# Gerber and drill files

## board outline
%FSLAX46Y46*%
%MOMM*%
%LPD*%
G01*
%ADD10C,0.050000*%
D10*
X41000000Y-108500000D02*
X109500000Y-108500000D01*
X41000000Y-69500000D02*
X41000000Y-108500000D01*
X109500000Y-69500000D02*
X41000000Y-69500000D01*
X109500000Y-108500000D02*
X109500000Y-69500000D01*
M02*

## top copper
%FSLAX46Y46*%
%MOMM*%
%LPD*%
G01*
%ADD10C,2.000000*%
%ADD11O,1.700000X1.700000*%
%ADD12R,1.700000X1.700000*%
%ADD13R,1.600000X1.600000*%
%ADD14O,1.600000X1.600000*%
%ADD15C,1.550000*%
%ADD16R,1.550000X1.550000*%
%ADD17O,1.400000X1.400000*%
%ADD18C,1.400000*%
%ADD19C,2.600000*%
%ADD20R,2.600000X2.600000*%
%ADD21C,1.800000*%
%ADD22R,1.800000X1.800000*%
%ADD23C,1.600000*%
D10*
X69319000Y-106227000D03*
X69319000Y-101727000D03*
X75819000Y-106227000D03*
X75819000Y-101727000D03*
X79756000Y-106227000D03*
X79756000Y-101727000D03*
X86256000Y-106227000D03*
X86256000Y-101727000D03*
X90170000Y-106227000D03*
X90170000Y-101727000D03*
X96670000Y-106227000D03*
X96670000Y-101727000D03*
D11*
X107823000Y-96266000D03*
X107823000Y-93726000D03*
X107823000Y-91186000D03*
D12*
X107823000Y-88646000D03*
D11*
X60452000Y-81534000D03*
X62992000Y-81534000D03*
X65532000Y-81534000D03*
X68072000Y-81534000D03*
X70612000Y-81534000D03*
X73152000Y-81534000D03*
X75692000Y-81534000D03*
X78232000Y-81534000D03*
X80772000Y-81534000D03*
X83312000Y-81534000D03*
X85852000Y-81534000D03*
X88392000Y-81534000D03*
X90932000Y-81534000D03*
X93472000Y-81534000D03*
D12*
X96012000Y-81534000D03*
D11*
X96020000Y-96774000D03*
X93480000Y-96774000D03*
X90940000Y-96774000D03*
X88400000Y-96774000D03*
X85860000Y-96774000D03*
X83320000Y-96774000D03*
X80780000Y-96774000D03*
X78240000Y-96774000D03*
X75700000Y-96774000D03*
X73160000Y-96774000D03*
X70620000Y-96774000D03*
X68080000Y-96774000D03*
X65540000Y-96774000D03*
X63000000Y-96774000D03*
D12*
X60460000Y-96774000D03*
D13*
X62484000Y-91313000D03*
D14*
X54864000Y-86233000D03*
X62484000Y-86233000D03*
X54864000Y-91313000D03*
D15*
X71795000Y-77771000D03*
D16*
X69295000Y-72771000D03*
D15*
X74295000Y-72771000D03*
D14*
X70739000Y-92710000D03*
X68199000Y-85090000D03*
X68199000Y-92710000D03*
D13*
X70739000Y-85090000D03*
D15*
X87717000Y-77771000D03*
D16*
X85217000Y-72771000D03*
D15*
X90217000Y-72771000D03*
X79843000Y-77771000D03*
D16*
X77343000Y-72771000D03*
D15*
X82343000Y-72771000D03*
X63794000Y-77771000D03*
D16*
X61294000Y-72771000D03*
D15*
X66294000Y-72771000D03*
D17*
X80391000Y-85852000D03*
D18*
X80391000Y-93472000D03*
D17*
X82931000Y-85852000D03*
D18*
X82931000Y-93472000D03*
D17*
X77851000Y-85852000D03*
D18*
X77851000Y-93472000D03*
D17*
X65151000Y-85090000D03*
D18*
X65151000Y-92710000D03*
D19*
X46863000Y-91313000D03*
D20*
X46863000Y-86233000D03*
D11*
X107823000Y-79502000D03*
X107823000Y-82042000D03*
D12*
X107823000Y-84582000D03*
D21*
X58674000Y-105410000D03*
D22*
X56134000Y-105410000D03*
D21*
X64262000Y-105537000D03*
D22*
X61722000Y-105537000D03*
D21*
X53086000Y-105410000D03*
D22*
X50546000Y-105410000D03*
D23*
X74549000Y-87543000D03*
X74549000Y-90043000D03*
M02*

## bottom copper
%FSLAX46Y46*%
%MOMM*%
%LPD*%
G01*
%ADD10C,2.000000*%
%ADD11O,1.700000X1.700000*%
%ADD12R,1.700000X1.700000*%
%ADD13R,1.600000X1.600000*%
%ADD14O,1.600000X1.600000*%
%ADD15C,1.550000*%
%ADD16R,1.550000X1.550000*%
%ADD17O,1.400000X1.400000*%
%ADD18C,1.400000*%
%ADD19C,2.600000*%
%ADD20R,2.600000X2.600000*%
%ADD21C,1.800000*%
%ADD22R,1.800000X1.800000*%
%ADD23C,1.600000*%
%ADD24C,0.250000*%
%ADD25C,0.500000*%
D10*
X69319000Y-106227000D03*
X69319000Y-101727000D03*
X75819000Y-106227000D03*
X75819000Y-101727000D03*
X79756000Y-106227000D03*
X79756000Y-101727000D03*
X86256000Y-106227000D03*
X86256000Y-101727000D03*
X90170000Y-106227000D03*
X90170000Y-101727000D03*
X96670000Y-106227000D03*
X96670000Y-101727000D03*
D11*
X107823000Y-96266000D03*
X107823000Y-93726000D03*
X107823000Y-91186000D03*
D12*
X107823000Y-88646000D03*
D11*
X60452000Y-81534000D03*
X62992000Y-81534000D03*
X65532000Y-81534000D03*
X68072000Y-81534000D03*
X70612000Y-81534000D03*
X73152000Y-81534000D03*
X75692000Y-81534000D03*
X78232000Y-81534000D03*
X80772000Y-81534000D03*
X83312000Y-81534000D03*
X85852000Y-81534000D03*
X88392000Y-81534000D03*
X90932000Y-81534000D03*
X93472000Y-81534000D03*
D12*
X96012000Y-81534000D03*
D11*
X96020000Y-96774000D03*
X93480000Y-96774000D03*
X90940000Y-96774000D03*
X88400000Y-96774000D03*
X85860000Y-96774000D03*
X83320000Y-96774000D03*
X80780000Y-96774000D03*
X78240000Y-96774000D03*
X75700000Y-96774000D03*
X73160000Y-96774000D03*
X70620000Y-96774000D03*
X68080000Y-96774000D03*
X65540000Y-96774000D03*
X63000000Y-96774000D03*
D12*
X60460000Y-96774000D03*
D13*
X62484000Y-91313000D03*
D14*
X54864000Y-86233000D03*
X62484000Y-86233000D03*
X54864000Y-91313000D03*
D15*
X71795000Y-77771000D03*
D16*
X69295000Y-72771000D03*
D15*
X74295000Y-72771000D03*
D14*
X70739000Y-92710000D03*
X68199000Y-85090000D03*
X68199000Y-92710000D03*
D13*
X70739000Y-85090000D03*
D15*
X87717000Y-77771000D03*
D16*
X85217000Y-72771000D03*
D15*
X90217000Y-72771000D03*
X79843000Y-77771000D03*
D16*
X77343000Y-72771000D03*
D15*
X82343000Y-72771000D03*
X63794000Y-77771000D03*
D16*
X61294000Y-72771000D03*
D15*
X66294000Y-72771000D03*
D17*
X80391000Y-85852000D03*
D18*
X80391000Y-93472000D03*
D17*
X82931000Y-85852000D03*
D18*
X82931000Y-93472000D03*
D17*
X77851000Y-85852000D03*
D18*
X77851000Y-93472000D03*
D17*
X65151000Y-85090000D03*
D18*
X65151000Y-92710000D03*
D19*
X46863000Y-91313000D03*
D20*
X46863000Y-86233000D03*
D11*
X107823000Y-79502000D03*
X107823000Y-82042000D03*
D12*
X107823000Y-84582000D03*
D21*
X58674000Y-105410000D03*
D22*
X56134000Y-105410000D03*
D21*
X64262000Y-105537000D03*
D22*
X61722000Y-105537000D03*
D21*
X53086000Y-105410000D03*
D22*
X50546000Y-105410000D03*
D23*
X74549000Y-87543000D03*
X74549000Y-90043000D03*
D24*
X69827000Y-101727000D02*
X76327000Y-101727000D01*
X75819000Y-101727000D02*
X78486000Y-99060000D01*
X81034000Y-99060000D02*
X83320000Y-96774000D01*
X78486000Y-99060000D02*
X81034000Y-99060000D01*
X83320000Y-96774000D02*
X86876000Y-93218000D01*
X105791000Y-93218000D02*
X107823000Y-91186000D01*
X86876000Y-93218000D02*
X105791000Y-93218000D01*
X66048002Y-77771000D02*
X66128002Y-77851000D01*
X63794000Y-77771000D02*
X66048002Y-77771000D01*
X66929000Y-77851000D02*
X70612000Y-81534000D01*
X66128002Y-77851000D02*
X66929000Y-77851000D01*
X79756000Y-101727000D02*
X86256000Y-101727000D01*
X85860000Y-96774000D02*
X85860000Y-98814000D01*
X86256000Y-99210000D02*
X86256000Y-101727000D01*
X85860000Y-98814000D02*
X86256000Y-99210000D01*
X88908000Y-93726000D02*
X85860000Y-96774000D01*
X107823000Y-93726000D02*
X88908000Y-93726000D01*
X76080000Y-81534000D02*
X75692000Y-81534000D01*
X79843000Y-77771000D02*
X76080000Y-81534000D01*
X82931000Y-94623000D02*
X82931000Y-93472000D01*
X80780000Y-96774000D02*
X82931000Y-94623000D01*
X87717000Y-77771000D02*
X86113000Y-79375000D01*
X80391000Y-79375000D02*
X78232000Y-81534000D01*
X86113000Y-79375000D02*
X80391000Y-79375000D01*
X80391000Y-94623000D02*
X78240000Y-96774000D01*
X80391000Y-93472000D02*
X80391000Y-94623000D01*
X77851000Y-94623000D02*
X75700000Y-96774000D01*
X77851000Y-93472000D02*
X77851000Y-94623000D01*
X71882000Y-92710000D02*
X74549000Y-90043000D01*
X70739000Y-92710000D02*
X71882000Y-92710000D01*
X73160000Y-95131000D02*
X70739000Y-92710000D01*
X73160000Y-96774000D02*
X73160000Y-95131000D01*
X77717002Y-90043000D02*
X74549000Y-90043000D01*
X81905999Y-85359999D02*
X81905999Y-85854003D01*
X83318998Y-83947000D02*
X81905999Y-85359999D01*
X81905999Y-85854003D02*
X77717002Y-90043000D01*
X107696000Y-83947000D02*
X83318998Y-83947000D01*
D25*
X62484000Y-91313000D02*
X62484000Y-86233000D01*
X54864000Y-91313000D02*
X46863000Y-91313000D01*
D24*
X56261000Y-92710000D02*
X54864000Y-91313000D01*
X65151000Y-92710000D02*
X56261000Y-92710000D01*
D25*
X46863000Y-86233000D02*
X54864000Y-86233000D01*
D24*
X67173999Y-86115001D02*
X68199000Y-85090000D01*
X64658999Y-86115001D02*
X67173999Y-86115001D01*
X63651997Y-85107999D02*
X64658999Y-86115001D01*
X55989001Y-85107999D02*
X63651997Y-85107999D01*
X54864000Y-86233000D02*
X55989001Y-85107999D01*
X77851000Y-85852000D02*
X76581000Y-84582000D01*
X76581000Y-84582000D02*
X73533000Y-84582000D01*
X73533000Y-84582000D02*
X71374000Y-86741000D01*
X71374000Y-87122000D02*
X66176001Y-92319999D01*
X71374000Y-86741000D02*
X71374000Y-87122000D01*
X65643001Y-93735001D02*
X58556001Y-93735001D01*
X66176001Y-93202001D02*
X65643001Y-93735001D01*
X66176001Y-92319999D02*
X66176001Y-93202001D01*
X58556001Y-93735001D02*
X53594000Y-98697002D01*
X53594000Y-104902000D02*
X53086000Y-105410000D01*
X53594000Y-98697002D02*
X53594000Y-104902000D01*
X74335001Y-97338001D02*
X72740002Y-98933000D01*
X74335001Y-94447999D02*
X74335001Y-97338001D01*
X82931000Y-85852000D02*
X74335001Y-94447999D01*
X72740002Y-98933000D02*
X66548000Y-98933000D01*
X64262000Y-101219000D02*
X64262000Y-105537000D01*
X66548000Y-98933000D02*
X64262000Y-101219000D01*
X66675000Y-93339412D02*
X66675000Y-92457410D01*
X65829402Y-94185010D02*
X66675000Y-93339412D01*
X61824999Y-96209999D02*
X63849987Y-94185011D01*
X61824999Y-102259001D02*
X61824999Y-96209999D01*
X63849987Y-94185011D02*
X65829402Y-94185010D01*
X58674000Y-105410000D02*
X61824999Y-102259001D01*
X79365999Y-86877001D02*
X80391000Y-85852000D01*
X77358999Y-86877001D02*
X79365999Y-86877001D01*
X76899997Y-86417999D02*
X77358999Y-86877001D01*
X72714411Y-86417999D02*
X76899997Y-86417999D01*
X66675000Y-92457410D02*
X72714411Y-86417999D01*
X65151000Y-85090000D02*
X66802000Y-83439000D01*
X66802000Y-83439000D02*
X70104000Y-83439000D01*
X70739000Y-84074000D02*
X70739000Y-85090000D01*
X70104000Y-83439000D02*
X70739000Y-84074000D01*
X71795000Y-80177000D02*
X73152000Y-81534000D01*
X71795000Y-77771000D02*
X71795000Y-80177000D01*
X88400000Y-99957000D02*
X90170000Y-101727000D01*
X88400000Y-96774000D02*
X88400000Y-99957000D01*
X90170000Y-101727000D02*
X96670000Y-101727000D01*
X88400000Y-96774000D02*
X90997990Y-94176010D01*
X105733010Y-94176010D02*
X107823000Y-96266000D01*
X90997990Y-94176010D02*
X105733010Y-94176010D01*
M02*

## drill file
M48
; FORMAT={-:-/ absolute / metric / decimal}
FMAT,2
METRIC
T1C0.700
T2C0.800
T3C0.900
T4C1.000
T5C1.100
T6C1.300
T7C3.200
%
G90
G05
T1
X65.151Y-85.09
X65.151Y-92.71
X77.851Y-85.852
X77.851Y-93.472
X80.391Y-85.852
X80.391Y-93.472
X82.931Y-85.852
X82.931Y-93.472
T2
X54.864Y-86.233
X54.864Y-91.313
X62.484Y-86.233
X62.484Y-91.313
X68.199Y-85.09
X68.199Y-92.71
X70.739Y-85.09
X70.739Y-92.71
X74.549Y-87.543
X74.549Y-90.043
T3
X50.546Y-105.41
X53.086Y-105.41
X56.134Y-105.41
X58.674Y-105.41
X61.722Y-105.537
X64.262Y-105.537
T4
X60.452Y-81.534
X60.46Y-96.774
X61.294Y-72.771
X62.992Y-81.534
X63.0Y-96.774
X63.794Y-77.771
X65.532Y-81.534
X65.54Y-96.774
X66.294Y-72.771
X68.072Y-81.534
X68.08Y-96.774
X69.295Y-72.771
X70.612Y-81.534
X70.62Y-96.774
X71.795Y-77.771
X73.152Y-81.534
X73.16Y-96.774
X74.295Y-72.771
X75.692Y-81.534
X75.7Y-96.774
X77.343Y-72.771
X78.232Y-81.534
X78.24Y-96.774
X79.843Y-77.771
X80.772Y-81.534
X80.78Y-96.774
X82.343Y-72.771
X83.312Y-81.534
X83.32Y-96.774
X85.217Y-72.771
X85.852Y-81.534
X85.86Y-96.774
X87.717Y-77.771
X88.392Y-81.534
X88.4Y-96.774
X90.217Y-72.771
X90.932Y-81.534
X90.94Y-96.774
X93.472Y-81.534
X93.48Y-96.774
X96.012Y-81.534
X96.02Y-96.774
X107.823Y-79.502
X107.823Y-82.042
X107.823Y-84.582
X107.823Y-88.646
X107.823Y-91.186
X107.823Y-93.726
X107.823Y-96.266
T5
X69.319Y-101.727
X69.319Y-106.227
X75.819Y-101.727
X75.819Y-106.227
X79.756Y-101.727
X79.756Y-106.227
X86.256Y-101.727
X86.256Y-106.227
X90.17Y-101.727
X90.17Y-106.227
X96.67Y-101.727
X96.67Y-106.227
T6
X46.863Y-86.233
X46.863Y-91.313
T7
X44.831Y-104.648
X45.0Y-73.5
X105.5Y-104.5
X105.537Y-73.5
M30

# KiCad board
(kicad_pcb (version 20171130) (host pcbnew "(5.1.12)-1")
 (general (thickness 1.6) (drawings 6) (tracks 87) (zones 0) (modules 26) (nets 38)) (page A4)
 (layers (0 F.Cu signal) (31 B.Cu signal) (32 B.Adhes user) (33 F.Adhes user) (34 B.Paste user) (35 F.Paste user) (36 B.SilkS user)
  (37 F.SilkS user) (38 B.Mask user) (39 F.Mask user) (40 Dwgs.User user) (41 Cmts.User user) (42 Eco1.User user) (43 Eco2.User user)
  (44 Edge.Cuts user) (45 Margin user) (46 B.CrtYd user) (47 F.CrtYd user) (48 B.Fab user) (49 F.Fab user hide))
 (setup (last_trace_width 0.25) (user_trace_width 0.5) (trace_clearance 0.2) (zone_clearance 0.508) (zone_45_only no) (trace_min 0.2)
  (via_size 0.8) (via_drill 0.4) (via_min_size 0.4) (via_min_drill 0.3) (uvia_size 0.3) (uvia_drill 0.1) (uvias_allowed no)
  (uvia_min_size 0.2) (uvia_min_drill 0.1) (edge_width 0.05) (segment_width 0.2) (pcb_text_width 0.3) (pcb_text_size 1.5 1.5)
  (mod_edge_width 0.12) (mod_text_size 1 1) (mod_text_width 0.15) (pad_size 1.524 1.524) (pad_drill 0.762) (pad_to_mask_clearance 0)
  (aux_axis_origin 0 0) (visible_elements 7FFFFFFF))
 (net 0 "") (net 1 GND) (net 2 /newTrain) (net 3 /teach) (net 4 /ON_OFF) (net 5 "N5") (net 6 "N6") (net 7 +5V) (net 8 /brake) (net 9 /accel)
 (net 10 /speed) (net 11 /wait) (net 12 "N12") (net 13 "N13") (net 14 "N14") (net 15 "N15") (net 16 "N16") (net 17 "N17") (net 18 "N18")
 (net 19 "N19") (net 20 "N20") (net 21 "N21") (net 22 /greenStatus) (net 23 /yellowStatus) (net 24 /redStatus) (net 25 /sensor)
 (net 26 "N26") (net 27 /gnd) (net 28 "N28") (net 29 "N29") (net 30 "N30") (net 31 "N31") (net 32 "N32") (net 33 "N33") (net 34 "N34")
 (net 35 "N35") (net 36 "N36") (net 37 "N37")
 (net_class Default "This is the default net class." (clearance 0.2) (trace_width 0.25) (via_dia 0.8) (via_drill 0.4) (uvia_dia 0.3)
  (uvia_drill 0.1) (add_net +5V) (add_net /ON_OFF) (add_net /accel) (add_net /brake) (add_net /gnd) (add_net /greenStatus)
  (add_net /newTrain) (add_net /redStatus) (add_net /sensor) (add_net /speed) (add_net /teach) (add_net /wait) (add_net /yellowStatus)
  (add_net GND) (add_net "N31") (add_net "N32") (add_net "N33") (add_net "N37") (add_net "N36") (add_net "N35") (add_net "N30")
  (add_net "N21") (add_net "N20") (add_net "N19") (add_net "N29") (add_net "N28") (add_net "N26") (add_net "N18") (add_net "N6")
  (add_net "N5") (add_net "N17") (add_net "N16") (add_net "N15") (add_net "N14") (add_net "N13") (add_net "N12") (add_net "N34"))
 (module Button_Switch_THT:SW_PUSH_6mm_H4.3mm (layer F.Cu) (at 75.819 106.227 180)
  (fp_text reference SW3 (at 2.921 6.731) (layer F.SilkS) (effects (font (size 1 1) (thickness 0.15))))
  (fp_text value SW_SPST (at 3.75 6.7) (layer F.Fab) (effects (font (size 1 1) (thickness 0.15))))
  (pad 1 thru_hole circle (at 6.5 0 270) (size 2 2) (drill 1.1) (layers *.Cu *.Mask) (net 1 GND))
  (pad 2 thru_hole circle (at 6.5 4.5 270) (size 2 2) (drill 1.1) (layers *.Cu *.Mask) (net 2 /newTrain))
  (pad 1 thru_hole circle (at 0 0 270) (size 2 2) (drill 1.1) (layers *.Cu *.Mask) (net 1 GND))
  (pad 2 thru_hole circle (at 0 4.5 270) (size 2 2) (drill 1.1) (layers *.Cu *.Mask) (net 2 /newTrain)))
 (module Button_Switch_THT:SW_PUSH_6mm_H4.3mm (layer F.Cu) (at 86.256 106.227 180)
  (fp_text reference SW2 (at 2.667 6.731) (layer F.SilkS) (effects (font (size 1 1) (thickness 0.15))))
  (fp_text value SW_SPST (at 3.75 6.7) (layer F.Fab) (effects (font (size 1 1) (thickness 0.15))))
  (pad 1 thru_hole circle (at 6.5 0 270) (size 2 2) (drill 1.1) (layers *.Cu *.Mask) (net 1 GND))
  (pad 2 thru_hole circle (at 6.5 4.5 270) (size 2 2) (drill 1.1) (layers *.Cu *.Mask) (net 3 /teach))
  (pad 1 thru_hole circle (at 0 0 270) (size 2 2) (drill 1.1) (layers *.Cu *.Mask) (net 1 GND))
  (pad 2 thru_hole circle (at 0 4.5 270) (size 2 2) (drill 1.1) (layers *.Cu *.Mask) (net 3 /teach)))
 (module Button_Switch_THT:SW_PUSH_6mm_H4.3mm (layer F.Cu) (at 96.67 106.227 180)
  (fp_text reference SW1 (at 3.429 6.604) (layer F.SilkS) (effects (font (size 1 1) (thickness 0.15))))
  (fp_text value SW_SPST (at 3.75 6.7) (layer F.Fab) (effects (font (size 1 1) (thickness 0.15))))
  (pad 1 thru_hole circle (at 6.5 0 270) (size 2 2) (drill 1.1) (layers *.Cu *.Mask) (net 1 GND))
  (pad 2 thru_hole circle (at 6.5 4.5 270) (size 2 2) (drill 1.1) (layers *.Cu *.Mask) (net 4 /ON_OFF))
  (pad 1 thru_hole circle (at 0 0 270) (size 2 2) (drill 1.1) (layers *.Cu *.Mask) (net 1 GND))
  (pad 2 thru_hole circle (at 0 4.5 270) (size 2 2) (drill 1.1) (layers *.Cu *.Mask) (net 4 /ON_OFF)))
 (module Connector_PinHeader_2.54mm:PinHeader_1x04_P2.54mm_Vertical (layer F.Cu) (at 107.823 88.646)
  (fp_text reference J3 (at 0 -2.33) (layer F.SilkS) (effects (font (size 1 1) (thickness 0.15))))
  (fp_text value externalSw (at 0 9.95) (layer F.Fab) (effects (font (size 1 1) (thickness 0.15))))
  (pad 4 thru_hole oval (at 0 7.62) (size 1.7 1.7) (drill 1) (layers *.Cu *.Mask) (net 4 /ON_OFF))
  (pad 3 thru_hole oval (at 0 5.08) (size 1.7 1.7) (drill 1) (layers *.Cu *.Mask) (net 3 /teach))
  (pad 2 thru_hole oval (at 0 2.54) (size 1.7 1.7) (drill 1) (layers *.Cu *.Mask) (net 2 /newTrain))
  (pad 1 thru_hole rect (at 0 0) (size 1.7 1.7) (drill 1) (layers *.Cu *.Mask) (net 1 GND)))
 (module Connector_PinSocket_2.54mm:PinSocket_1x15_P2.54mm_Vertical (layer F.Cu) (at 96.012 81.534 270)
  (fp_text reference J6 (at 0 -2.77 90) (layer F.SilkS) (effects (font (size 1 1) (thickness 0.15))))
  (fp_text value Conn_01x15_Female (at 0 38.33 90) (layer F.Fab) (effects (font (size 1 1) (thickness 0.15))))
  (pad 15 thru_hole oval (at 0 35.56 270) (size 1.7 1.7) (drill 1) (layers *.Cu *.Mask) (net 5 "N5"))
  (pad 14 thru_hole oval (at 0 33.02 270) (size 1.7 1.7) (drill 1) (layers *.Cu *.Mask) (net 1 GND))
  (pad 13 thru_hole oval (at 0 30.48 270) (size 1.7 1.7) (drill 1) (layers *.Cu *.Mask) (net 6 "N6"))
  (pad 12 thru_hole oval (at 0 27.94 270) (size 1.7 1.7) (drill 1) (layers *.Cu *.Mask) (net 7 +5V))
  (pad 11 thru_hole oval (at 0 25.4 270) (size 1.7 1.7) (drill 1) (layers *.Cu *.Mask) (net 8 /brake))
  (pad 10 thru_hole oval (at 0 22.86 270) (size 1.7 1.7) (drill 1) (layers *.Cu *.Mask) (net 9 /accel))
  (pad 9 thru_hole oval (at 0 20.32 270) (size 1.7 1.7) (drill 1) (layers *.Cu *.Mask) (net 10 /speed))
  (pad 8 thru_hole oval (at 0 17.78 270) (size 1.7 1.7) (drill 1) (layers *.Cu *.Mask) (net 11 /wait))
  (pad 7 thru_hole oval (at 0 15.24 270) (size 1.7 1.7) (drill 1) (layers *.Cu *.Mask) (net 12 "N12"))
  (pad 6 thru_hole oval (at 0 12.7 270) (size 1.7 1.7) (drill 1) (layers *.Cu *.Mask) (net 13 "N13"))
  (pad 5 thru_hole oval (at 0 10.16 270) (size 1.7 1.7) (drill 1) (layers *.Cu *.Mask) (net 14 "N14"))
  (pad 4 thru_hole oval (at 0 7.62 270) (size 1.7 1.7) (drill 1) (layers *.Cu *.Mask) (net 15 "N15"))
  (pad 3 thru_hole oval (at 0 5.08 270) (size 1.7 1.7) (drill 1) (layers *.Cu *.Mask) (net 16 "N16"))
  (pad 2 thru_hole oval (at 0 2.54 270) (size 1.7 1.7) (drill 1) (layers *.Cu *.Mask) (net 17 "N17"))
  (pad 1 thru_hole rect (at 0 0 270) (size 1.7 1.7) (drill 1) (layers *.Cu *.Mask) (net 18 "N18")))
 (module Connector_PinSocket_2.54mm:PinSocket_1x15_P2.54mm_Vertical (layer F.Cu) (at 60.46 96.774 90)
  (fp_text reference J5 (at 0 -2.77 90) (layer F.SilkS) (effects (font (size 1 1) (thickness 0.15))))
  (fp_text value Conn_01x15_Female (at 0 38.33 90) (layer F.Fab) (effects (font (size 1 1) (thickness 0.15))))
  (pad 15 thru_hole oval (at 0 35.56 90) (size 1.7 1.7) (drill 1) (layers *.Cu *.Mask) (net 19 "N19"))
  (pad 14 thru_hole oval (at 0 33.02 90) (size 1.7 1.7) (drill 1) (layers *.Cu *.Mask) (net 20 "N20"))
  (pad 13 thru_hole oval (at 0 30.48 90) (size 1.7 1.7) (drill 1) (layers *.Cu *.Mask) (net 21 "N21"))
  (pad 12 thru_hole oval (at 0 27.94 90) (size 1.7 1.7) (drill 1) (layers *.Cu *.Mask) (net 4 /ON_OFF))
  (pad 11 thru_hole oval (at 0 25.4 90) (size 1.7 1.7) (drill 1) (layers *.Cu *.Mask) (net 3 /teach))
  (pad 10 thru_hole oval (at 0 22.86 90) (size 1.7 1.7) (drill 1) (layers *.Cu *.Mask) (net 2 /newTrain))
  (pad 9 thru_hole oval (at 0 20.32 90) (size 1.7 1.7) (drill 1) (layers *.Cu *.Mask) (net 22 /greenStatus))
  (pad 8 thru_hole oval (at 0 17.78 90) (size 1.7 1.7) (drill 1) (layers *.Cu *.Mask) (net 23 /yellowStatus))
  (pad 7 thru_hole oval (at 0 15.24 90) (size 1.7 1.7) (drill 1) (layers *.Cu *.Mask) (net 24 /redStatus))
  (pad 6 thru_hole oval (at 0 12.7 90) (size 1.7 1.7) (drill 1) (layers *.Cu *.Mask) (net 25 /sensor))
  (pad 5 thru_hole oval (at 0 10.16 90) (size 1.7 1.7) (drill 1) (layers *.Cu *.Mask) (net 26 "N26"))
  (pad 4 thru_hole oval (at 0 7.62 90) (size 1.7 1.7) (drill 1) (layers *.Cu *.Mask) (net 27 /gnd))
  (pad 3 thru_hole oval (at 0 5.08 90) (size 1.7 1.7) (drill 1) (layers *.Cu *.Mask) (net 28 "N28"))
  (pad 2 thru_hole oval (at 0 2.54 90) (size 1.7 1.7) (drill 1) (layers *.Cu *.Mask) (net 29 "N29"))
  (pad 1 thru_hole rect (at 0 0 90) (size 1.7 1.7) (drill 1) (layers *.Cu *.Mask) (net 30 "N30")))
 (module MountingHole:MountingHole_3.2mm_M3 (layer F.Cu) (at 44.831 104.648)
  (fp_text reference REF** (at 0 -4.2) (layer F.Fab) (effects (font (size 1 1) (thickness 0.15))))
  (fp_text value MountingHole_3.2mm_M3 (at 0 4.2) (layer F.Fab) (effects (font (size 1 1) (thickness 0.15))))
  (pad 1 np_thru_hole circle (at 0 0) (size 3.2 3.2) (drill 3.2) (layers *.Cu *.Mask)))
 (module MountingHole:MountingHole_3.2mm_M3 (layer F.Cu) (at 45 73.5)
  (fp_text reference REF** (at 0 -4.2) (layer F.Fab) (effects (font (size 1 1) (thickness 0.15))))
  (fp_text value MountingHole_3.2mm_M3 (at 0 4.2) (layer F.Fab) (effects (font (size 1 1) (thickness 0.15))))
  (pad 1 np_thru_hole circle (at 0 0) (size 3.2 3.2) (drill 3.2) (layers *.Cu *.Mask)))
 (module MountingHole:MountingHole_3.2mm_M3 (layer F.Cu) (at 105.537 73.5)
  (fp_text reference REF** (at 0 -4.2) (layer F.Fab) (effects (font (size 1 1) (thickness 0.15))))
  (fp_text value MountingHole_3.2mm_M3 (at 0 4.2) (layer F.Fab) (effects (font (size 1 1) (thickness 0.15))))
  (pad 1 np_thru_hole circle (at 0 0) (size 3.2 3.2) (drill 3.2) (layers *.Cu *.Mask)))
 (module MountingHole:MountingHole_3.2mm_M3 (layer F.Cu) (at 105.5 104.5)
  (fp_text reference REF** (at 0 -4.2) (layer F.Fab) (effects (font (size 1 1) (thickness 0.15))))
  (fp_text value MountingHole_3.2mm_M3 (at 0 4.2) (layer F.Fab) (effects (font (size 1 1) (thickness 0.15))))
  (pad 1 np_thru_hole circle (at 0 0) (size 3.2 3.2) (drill 3.2) (layers *.Cu *.Mask)))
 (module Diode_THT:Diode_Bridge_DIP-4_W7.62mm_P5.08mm (layer F.Cu) (at 62.484 91.313 180)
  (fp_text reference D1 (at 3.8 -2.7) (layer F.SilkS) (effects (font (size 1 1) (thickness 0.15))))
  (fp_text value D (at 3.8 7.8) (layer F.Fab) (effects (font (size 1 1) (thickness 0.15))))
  (pad 1 thru_hole rect (at 0 0 180) (size 1.6 1.6) (drill 0.8) (layers *.Cu *.Mask) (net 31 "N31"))
  (pad 3 thru_hole oval (at 7.62 5.08 180) (size 1.6 1.6) (drill 0.8) (layers *.Cu *.Mask) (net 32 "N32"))
  (pad 2 thru_hole oval (at 0 5.08 180) (size 1.6 1.6) (drill 0.8) (layers *.Cu *.Mask) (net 31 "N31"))
  (pad 4 thru_hole oval (at 7.62 0 180) (size 1.6 1.6) (drill 0.8) (layers *.Cu *.Mask) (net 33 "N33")))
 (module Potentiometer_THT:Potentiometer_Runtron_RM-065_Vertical (layer F.Cu) (at 69.295 72.771)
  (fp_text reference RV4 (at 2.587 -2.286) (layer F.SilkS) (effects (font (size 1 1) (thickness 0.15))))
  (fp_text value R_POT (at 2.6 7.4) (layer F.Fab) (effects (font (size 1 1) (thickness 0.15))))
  (pad 2 thru_hole circle (at 2.5 5) (size 1.55 1.55) (drill 1) (layers *.Cu *.Mask) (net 9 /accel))
  (pad 1 thru_hole rect (at 0 0) (size 1.55 1.55) (drill 1) (layers *.Cu *.Mask) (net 1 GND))
  (pad 3 thru_hole circle (at 5 0) (size 1.55 1.55) (drill 1) (layers *.Cu *.Mask) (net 7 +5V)))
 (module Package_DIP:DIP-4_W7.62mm (layer F.Cu) (at 70.739 85.09 270)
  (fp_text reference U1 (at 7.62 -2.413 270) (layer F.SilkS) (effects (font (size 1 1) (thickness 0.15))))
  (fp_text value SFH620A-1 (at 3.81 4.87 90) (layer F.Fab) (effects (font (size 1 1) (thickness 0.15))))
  (pad 4 thru_hole oval (at 7.62 0 270) (size 1.6 1.6) (drill 0.8) (layers *.Cu *.Mask) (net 25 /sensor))
  (pad 2 thru_hole oval (at 0 2.54 270) (size 1.6 1.6) (drill 0.8) (layers *.Cu *.Mask) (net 32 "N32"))
  (pad 3 thru_hole oval (at 7.62 2.54 270) (size 1.6 1.6) (drill 0.8) (layers *.Cu *.Mask) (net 1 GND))
  (pad 1 thru_hole rect (at 0 0 270) (size 1.6 1.6) (drill 0.8) (layers *.Cu *.Mask) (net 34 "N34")))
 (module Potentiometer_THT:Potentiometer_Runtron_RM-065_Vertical (layer F.Cu) (at 85.217 72.771)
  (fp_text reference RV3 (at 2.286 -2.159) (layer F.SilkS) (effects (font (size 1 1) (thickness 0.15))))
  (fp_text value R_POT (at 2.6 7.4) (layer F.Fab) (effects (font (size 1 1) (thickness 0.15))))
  (pad 2 thru_hole circle (at 2.5 5) (size 1.55 1.55) (drill 1) (layers *.Cu *.Mask) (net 11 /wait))
  (pad 1 thru_hole rect (at 0 0) (size 1.55 1.55) (drill 1) (layers *.Cu *.Mask) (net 1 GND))
  (pad 3 thru_hole circle (at 5 0) (size 1.55 1.55) (drill 1) (layers *.Cu *.Mask) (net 7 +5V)))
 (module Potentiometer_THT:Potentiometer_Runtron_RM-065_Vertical (layer F.Cu) (at 77.343 72.771)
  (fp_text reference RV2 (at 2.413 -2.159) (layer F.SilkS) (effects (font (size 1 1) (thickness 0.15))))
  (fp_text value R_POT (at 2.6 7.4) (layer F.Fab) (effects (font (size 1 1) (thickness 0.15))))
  (pad 2 thru_hole circle (at 2.5 5) (size 1.55 1.55) (drill 1) (layers *.Cu *.Mask) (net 10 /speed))
  (pad 1 thru_hole rect (at 0 0) (size 1.55 1.55) (drill 1) (layers *.Cu *.Mask) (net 1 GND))
  (pad 3 thru_hole circle (at 5 0) (size 1.55 1.55) (drill 1) (layers *.Cu *.Mask) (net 7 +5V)))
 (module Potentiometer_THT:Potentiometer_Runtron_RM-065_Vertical (layer F.Cu) (at 61.294 72.771)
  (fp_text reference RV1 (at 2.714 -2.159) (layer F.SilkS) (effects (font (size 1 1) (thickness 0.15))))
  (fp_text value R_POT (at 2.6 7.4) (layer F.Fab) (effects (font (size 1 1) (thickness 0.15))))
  (pad 2 thru_hole circle (at 2.5 5) (size 1.55 1.55) (drill 1) (layers *.Cu *.Mask) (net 8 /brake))
  (pad 1 thru_hole rect (at 0 0) (size 1.55 1.55) (drill 1) (layers *.Cu *.Mask) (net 1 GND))
  (pad 3 thru_hole circle (at 5 0) (size 1.55 1.55) (drill 1) (layers *.Cu *.Mask) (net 7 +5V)))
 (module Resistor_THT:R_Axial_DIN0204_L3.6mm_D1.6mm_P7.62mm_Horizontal (layer F.Cu) (at 80.391 93.472 90)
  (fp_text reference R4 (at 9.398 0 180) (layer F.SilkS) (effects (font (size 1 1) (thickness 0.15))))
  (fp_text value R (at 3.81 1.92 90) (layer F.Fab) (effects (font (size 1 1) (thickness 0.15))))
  (pad 2 thru_hole oval (at 7.62 0 90) (size 1.4 1.4) (drill 0.7) (layers *.Cu *.Mask) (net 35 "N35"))
  (pad 1 thru_hole circle (at 0 0 90) (size 1.4 1.4) (drill 0.7) (layers *.Cu *.Mask) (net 23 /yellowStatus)))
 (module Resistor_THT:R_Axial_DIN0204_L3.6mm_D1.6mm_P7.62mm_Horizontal (layer F.Cu) (at 82.931 93.472 90)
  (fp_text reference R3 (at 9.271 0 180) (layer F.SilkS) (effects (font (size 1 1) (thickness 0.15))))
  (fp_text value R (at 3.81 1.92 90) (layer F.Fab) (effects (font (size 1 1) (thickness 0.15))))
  (pad 2 thru_hole oval (at 7.62 0 90) (size 1.4 1.4) (drill 0.7) (layers *.Cu *.Mask) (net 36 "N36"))
  (pad 1 thru_hole circle (at 0 0 90) (size 1.4 1.4) (drill 0.7) (layers *.Cu *.Mask) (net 22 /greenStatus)))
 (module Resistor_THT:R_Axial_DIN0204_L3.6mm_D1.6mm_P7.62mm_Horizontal (layer F.Cu) (at 77.851 93.472 90)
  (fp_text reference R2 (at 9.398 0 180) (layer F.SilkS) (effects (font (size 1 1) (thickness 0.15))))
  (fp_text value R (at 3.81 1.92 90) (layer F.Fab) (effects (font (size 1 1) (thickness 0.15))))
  (pad 2 thru_hole oval (at 7.62 0 90) (size 1.4 1.4) (drill 0.7) (layers *.Cu *.Mask) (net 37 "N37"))
  (pad 1 thru_hole circle (at 0 0 90) (size 1.4 1.4) (drill 0.7) (layers *.Cu *.Mask) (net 24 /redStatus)))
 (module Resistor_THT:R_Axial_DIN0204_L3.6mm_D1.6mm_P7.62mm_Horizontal (layer F.Cu) (at 65.151 92.71 90)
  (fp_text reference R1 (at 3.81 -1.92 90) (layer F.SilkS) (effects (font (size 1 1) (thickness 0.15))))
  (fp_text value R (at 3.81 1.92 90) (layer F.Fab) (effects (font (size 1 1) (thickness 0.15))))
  (pad 2 thru_hole oval (at 7.62 0 90) (size 1.4 1.4) (drill 0.7) (layers *.Cu *.Mask) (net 34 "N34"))
  (pad 1 thru_hole circle (at 0 0 90) (size 1.4 1.4) (drill 0.7) (layers *.Cu *.Mask) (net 33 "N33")))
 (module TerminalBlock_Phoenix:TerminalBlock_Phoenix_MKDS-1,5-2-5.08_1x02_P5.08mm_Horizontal (layer F.Cu) (at 46.863 86.233 270)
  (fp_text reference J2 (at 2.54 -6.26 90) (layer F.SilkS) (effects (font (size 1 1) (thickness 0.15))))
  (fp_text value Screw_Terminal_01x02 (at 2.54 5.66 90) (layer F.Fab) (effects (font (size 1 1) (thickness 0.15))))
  (pad 2 thru_hole circle (at 5.08 0 270) (size 2.6 2.6) (drill 1.3) (layers *.Cu *.Mask) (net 33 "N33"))
  (pad 1 thru_hole rect (at 0 0 270) (size 2.6 2.6) (drill 1.3) (layers *.Cu *.Mask) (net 32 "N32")))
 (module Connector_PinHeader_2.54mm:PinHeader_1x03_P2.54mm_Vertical (layer F.Cu) (at 107.823 84.582 180)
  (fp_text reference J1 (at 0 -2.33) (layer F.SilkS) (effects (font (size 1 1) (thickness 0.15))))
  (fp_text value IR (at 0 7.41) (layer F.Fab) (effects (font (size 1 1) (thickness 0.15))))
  (pad 3 thru_hole oval (at 0 5.08 180) (size 1.7 1.7) (drill 1) (layers *.Cu *.Mask) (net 1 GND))
  (pad 2 thru_hole oval (at 0 2.54 180) (size 1.7 1.7) (drill 1) (layers *.Cu *.Mask) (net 7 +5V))
  (pad 1 thru_hole rect (at 0 0 180) (size 1.7 1.7) (drill 1) (layers *.Cu *.Mask) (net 25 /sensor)))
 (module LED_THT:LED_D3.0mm (layer F.Cu) (at 56.134 105.41)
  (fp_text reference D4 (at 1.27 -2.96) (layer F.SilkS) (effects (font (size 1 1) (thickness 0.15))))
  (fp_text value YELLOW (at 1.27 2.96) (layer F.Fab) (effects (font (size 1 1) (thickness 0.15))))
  (pad 2 thru_hole circle (at 2.54 0) (size 1.8 1.8) (drill 0.9) (layers *.Cu *.Mask) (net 35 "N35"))
  (pad 1 thru_hole rect (at 0 0) (size 1.8 1.8) (drill 0.9) (layers *.Cu *.Mask) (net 1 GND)))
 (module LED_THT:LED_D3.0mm (layer F.Cu) (at 61.722 105.537)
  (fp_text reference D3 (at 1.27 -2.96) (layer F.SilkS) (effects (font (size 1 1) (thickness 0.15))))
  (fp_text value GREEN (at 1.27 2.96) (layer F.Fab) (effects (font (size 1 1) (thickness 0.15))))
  (pad 2 thru_hole circle (at 2.54 0) (size 1.8 1.8) (drill 0.9) (layers *.Cu *.Mask) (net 36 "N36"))
  (pad 1 thru_hole rect (at 0 0) (size 1.8 1.8) (drill 0.9) (layers *.Cu *.Mask) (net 1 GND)))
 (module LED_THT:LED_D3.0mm (layer F.Cu) (at 50.546 105.41)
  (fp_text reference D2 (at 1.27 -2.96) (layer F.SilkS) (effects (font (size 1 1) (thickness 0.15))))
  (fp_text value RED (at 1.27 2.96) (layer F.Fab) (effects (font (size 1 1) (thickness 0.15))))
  (pad 2 thru_hole circle (at 2.54 0) (size 1.8 1.8) (drill 0.9) (layers *.Cu *.Mask) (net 37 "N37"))
  (pad 1 thru_hole rect (at 0 0) (size 1.8 1.8) (drill 0.9) (layers *.Cu *.Mask) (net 1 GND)))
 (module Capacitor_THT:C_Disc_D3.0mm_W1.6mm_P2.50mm (layer F.Cu) (at 74.549 90.043 90)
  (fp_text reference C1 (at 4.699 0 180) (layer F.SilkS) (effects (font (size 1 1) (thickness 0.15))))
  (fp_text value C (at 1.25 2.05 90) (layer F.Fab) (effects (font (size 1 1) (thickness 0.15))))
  (pad 2 thru_hole circle (at 2.5 0 90) (size 1.6 1.6) (drill 0.8) (layers *.Cu *.Mask) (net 1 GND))
  (pad 1 thru_hole circle (at 0 0 90) (size 1.6 1.6) (drill 0.8) (layers *.Cu *.Mask) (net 25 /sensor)))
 (gr_line (start 41 108.5) (end 109.5 108.5) (layer Edge.Cuts) (width 0.05))
 (gr_line (start 41 69.5) (end 41 108.5) (layer Edge.Cuts) (width 0.05))
 (gr_line (start 109.5 69.5) (end 41 69.5) (layer Edge.Cuts) (width 0.05))
 (gr_line (start 109.5 108.5) (end 109.5 69.5) (layer Edge.Cuts) (width 0.05))
 (segment (start 69.827 101.727) (end 76.327 101.727) (width 0.25) (layer B.Cu) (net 2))
 (segment (start 75.819 101.727) (end 78.486 99.06) (width 0.25) (layer B.Cu) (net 2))
 (segment (start 81.034 99.06) (end 83.32 96.774) (width 0.25) (layer B.Cu) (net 2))
 (segment (start 78.486 99.06) (end 81.034 99.06) (width 0.25) (layer B.Cu) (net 2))
 (segment (start 83.32 96.774) (end 86.876 93.218) (width 0.25) (layer B.Cu) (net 2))
 (segment (start 105.791 93.218) (end 107.823 91.186) (width 0.25) (layer B.Cu) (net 2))
 (segment (start 86.876 93.218) (end 105.791 93.218) (width 0.25) (layer B.Cu) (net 2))
 (segment (start 66.048002 77.771) (end 66.128002 77.851) (width 0.25) (layer B.Cu) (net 8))
 (segment (start 63.794 77.771) (end 66.048002 77.771) (width 0.25) (layer B.Cu) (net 8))
 (segment (start 66.929 77.851) (end 70.612 81.534) (width 0.25) (layer B.Cu) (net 8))
 (segment (start 66.128002 77.851) (end 66.929 77.851) (width 0.25) (layer B.Cu) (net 8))
 (segment (start 79.756 101.727) (end 86.256 101.727) (width 0.25) (layer B.Cu) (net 3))
 (segment (start 85.86 96.774) (end 85.86 98.814) (width 0.25) (layer B.Cu) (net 3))
 (segment (start 86.256 99.21) (end 86.256 101.727) (width 0.25) (layer B.Cu) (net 3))
 (segment (start 85.86 98.814) (end 86.256 99.21) (width 0.25) (layer B.Cu) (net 3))
 (segment (start 88.908 93.726) (end 85.86 96.774) (width 0.25) (layer B.Cu) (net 3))
 (segment (start 107.823 93.726) (end 88.908 93.726) (width 0.25) (layer B.Cu) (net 3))
 (segment (start 76.08 81.534) (end 75.692 81.534) (width 0.25) (layer B.Cu) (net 10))
 (segment (start 79.843 77.771) (end 76.08 81.534) (width 0.25) (layer B.Cu) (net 10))
 (segment (start 82.931 94.623) (end 82.931 93.472) (width 0.25) (layer B.Cu) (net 22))
 (segment (start 80.78 96.774) (end 82.931 94.623) (width 0.25) (layer B.Cu) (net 22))
 (segment (start 87.717 77.771) (end 86.113 79.375) (width 0.25) (layer B.Cu) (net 11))
 (segment (start 80.391 79.375) (end 78.232 81.534) (width 0.25) (layer B.Cu) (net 11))
 (segment (start 86.113 79.375) (end 80.391 79.375) (width 0.25) (layer B.Cu) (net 11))
 (segment (start 80.391 94.623) (end 78.24 96.774) (width 0.25) (layer B.Cu) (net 23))
 (segment (start 80.391 93.472) (end 80.391 94.623) (width 0.25) (layer B.Cu) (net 23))
 (segment (start 77.851 94.623) (end 75.7 96.774) (width 0.25) (layer B.Cu) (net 24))
 (segment (start 77.851 93.472) (end 77.851 94.623) (width 0.25) (layer B.Cu) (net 24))
 (segment (start 71.882 92.71) (end 74.549 90.043) (width 0.25) (layer B.Cu) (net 25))
 (segment (start 70.739 92.71) (end 71.882 92.71) (width 0.25) (layer B.Cu) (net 25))
 (segment (start 73.16 95.131) (end 70.739 92.71) (width 0.25) (layer B.Cu) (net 25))
 (segment (start 73.16 96.774) (end 73.16 95.131) (width 0.25) (layer B.Cu) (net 25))
 (segment (start 77.717002 90.043) (end 74.549 90.043) (width 0.25) (layer B.Cu) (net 25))
 (segment (start 81.905999 85.359999) (end 81.905999 85.854003) (width 0.25) (layer B.Cu) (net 25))
 (segment (start 83.318998 83.947) (end 81.905999 85.359999) (width 0.25) (layer B.Cu) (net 25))
 (segment (start 81.905999 85.854003) (end 77.717002 90.043) (width 0.25) (layer B.Cu) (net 25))
 (segment (start 107.696 83.947) (end 83.318998 83.947) (width 0.25) (layer B.Cu) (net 25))
 (segment (start 62.484 91.313) (end 62.484 86.233) (width 0.5) (layer B.Cu) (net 31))
 (segment (start 54.864 91.313) (end 46.863 91.313) (width 0.5) (layer B.Cu) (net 33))
 (segment (start 56.261 92.71) (end 54.864 91.313) (width 0.25) (layer B.Cu) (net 33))
 (segment (start 65.151 92.71) (end 56.261 92.71) (width 0.25) (layer B.Cu) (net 33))
 (segment (start 46.863 86.233) (end 54.864 86.233) (width 0.5) (layer B.Cu) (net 32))
 (segment (start 67.173999 86.115001) (end 68.199 85.09) (width 0.25) (layer B.Cu) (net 32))
 (segment (start 64.658999 86.115001) (end 67.173999 86.115001) (width 0.25) (layer B.Cu) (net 32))
 (segment (start 63.651997 85.107999) (end 64.658999 86.115001) (width 0.25) (layer B.Cu) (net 32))
 (segment (start 55.989001 85.107999) (end 63.651997 85.107999) (width 0.25) (layer B.Cu) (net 32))
 (segment (start 54.864 86.233) (end 55.989001 85.107999) (width 0.25) (layer B.Cu) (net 32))
 (segment (start 77.851 85.852) (end 76.581 84.582) (width 0.25) (layer B.Cu) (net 37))
 (segment (start 76.581 84.582) (end 73.533 84.582) (width 0.25) (layer B.Cu) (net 37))
 (segment (start 73.533 84.582) (end 71.374 86.741) (width 0.25) (layer B.Cu) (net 37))
 (segment (start 71.374 87.122) (end 66.176001 92.319999) (width 0.25) (layer B.Cu) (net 37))
 (segment (start 71.374 86.741) (end 71.374 87.122) (width 0.25) (layer B.Cu) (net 37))
 (segment (start 65.643001 93.735001) (end 58.556001 93.735001) (width 0.25) (layer B.Cu) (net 37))
 (segment (start 66.176001 93.202001) (end 65.643001 93.735001) (width 0.25) (layer B.Cu) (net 37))
 (segment (start 66.176001 92.319999) (end 66.176001 93.202001) (width 0.25) (layer B.Cu) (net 37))
 (segment (start 58.556001 93.735001) (end 53.594 98.697002) (width 0.25) (layer B.Cu) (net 37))
 (segment (start 53.594 104.902) (end 53.086 105.41) (width 0.25) (layer B.Cu) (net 37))
 (segment (start 53.594 98.697002) (end 53.594 104.902) (width 0.25) (layer B.Cu) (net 37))
 (segment (start 74.335001 97.338001) (end 72.740002 98.933) (width 0.25) (layer B.Cu) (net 36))
 (segment (start 74.335001 94.447999) (end 74.335001 97.338001) (width 0.25) (layer B.Cu) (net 36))
 (segment (start 82.931 85.852) (end 74.335001 94.447999) (width 0.25) (layer B.Cu) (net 36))
 (segment (start 72.740002 98.933) (end 66.548 98.933) (width 0.25) (layer B.Cu) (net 36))
 (segment (start 64.262 101.219) (end 64.262 105.537) (width 0.25) (layer B.Cu) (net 36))
 (segment (start 66.548 98.933) (end 64.262 101.219) (width 0.25) (layer B.Cu) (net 36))
 (segment (start 66.675 93.339412) (end 66.675 92.45741) (width 0.25) (layer B.Cu) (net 35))
 (segment (start 65.829402 94.18501) (end 66.675 93.339412) (width 0.25) (layer B.Cu) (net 35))
 (segment (start 61.824999 96.209999) (end 63.849987 94.185011) (width 0.25) (layer B.Cu) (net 35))
 (segment (start 61.824999 102.259001) (end 61.824999 96.209999) (width 0.25) (layer B.Cu) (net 35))
 (segment (start 63.849987 94.185011) (end 65.829402 94.18501) (width 0.25) (layer B.Cu) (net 35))
 (segment (start 58.674 105.41) (end 61.824999 102.259001) (width 0.25) (layer B.Cu) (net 35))
 (segment (start 79.365999 86.877001) (end 80.391 85.852) (width 0.25) (layer B.Cu) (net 35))
 (segment (start 77.358999 86.877001) (end 79.365999 86.877001) (width 0.25) (layer B.Cu) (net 35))
 (segment (start 76.899997 86.417999) (end 77.358999 86.877001) (width 0.25) (layer B.Cu) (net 35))
 (segment (start 72.714411 86.417999) (end 76.899997 86.417999) (width 0.25) (layer B.Cu) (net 35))
 (segment (start 66.675 92.45741) (end 72.714411 86.417999) (width 0.25) (layer B.Cu) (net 35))
 (segment (start 65.151 85.09) (end 66.802 83.439) (width 0.25) (layer B.Cu) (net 34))
 (segment (start 66.802 83.439) (end 70.104 83.439) (width 0.25) (layer B.Cu) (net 34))
 (segment (start 70.739 84.074) (end 70.739 85.09) (width 0.25) (layer B.Cu) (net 34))
 (segment (start 70.104 83.439) (end 70.739 84.074) (width 0.25) (layer B.Cu) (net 34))
 (segment (start 71.795 80.177) (end 73.152 81.534) (width 0.25) (layer B.Cu) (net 9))
 (segment (start 71.795 77.771) (end 71.795 80.177) (width 0.25) (layer B.Cu) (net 9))
 (segment (start 88.4 99.957) (end 90.17 101.727) (width 0.25) (layer B.Cu) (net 4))
 (segment (start 88.4 96.774) (end 88.4 99.957) (width 0.25) (layer B.Cu) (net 4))
 (segment (start 90.17 101.727) (end 96.67 101.727) (width 0.25) (layer B.Cu) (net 4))
 (segment (start 88.4 96.774) (end 90.99799 94.17601) (width 0.25) (layer B.Cu) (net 4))
 (segment (start 105.73301 94.17601) (end 107.823 96.266) (width 0.25) (layer B.Cu) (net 4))
 (segment (start 90.99799 94.17601) (end 105.73301 94.17601) (width 0.25) (layer B.Cu) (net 4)))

